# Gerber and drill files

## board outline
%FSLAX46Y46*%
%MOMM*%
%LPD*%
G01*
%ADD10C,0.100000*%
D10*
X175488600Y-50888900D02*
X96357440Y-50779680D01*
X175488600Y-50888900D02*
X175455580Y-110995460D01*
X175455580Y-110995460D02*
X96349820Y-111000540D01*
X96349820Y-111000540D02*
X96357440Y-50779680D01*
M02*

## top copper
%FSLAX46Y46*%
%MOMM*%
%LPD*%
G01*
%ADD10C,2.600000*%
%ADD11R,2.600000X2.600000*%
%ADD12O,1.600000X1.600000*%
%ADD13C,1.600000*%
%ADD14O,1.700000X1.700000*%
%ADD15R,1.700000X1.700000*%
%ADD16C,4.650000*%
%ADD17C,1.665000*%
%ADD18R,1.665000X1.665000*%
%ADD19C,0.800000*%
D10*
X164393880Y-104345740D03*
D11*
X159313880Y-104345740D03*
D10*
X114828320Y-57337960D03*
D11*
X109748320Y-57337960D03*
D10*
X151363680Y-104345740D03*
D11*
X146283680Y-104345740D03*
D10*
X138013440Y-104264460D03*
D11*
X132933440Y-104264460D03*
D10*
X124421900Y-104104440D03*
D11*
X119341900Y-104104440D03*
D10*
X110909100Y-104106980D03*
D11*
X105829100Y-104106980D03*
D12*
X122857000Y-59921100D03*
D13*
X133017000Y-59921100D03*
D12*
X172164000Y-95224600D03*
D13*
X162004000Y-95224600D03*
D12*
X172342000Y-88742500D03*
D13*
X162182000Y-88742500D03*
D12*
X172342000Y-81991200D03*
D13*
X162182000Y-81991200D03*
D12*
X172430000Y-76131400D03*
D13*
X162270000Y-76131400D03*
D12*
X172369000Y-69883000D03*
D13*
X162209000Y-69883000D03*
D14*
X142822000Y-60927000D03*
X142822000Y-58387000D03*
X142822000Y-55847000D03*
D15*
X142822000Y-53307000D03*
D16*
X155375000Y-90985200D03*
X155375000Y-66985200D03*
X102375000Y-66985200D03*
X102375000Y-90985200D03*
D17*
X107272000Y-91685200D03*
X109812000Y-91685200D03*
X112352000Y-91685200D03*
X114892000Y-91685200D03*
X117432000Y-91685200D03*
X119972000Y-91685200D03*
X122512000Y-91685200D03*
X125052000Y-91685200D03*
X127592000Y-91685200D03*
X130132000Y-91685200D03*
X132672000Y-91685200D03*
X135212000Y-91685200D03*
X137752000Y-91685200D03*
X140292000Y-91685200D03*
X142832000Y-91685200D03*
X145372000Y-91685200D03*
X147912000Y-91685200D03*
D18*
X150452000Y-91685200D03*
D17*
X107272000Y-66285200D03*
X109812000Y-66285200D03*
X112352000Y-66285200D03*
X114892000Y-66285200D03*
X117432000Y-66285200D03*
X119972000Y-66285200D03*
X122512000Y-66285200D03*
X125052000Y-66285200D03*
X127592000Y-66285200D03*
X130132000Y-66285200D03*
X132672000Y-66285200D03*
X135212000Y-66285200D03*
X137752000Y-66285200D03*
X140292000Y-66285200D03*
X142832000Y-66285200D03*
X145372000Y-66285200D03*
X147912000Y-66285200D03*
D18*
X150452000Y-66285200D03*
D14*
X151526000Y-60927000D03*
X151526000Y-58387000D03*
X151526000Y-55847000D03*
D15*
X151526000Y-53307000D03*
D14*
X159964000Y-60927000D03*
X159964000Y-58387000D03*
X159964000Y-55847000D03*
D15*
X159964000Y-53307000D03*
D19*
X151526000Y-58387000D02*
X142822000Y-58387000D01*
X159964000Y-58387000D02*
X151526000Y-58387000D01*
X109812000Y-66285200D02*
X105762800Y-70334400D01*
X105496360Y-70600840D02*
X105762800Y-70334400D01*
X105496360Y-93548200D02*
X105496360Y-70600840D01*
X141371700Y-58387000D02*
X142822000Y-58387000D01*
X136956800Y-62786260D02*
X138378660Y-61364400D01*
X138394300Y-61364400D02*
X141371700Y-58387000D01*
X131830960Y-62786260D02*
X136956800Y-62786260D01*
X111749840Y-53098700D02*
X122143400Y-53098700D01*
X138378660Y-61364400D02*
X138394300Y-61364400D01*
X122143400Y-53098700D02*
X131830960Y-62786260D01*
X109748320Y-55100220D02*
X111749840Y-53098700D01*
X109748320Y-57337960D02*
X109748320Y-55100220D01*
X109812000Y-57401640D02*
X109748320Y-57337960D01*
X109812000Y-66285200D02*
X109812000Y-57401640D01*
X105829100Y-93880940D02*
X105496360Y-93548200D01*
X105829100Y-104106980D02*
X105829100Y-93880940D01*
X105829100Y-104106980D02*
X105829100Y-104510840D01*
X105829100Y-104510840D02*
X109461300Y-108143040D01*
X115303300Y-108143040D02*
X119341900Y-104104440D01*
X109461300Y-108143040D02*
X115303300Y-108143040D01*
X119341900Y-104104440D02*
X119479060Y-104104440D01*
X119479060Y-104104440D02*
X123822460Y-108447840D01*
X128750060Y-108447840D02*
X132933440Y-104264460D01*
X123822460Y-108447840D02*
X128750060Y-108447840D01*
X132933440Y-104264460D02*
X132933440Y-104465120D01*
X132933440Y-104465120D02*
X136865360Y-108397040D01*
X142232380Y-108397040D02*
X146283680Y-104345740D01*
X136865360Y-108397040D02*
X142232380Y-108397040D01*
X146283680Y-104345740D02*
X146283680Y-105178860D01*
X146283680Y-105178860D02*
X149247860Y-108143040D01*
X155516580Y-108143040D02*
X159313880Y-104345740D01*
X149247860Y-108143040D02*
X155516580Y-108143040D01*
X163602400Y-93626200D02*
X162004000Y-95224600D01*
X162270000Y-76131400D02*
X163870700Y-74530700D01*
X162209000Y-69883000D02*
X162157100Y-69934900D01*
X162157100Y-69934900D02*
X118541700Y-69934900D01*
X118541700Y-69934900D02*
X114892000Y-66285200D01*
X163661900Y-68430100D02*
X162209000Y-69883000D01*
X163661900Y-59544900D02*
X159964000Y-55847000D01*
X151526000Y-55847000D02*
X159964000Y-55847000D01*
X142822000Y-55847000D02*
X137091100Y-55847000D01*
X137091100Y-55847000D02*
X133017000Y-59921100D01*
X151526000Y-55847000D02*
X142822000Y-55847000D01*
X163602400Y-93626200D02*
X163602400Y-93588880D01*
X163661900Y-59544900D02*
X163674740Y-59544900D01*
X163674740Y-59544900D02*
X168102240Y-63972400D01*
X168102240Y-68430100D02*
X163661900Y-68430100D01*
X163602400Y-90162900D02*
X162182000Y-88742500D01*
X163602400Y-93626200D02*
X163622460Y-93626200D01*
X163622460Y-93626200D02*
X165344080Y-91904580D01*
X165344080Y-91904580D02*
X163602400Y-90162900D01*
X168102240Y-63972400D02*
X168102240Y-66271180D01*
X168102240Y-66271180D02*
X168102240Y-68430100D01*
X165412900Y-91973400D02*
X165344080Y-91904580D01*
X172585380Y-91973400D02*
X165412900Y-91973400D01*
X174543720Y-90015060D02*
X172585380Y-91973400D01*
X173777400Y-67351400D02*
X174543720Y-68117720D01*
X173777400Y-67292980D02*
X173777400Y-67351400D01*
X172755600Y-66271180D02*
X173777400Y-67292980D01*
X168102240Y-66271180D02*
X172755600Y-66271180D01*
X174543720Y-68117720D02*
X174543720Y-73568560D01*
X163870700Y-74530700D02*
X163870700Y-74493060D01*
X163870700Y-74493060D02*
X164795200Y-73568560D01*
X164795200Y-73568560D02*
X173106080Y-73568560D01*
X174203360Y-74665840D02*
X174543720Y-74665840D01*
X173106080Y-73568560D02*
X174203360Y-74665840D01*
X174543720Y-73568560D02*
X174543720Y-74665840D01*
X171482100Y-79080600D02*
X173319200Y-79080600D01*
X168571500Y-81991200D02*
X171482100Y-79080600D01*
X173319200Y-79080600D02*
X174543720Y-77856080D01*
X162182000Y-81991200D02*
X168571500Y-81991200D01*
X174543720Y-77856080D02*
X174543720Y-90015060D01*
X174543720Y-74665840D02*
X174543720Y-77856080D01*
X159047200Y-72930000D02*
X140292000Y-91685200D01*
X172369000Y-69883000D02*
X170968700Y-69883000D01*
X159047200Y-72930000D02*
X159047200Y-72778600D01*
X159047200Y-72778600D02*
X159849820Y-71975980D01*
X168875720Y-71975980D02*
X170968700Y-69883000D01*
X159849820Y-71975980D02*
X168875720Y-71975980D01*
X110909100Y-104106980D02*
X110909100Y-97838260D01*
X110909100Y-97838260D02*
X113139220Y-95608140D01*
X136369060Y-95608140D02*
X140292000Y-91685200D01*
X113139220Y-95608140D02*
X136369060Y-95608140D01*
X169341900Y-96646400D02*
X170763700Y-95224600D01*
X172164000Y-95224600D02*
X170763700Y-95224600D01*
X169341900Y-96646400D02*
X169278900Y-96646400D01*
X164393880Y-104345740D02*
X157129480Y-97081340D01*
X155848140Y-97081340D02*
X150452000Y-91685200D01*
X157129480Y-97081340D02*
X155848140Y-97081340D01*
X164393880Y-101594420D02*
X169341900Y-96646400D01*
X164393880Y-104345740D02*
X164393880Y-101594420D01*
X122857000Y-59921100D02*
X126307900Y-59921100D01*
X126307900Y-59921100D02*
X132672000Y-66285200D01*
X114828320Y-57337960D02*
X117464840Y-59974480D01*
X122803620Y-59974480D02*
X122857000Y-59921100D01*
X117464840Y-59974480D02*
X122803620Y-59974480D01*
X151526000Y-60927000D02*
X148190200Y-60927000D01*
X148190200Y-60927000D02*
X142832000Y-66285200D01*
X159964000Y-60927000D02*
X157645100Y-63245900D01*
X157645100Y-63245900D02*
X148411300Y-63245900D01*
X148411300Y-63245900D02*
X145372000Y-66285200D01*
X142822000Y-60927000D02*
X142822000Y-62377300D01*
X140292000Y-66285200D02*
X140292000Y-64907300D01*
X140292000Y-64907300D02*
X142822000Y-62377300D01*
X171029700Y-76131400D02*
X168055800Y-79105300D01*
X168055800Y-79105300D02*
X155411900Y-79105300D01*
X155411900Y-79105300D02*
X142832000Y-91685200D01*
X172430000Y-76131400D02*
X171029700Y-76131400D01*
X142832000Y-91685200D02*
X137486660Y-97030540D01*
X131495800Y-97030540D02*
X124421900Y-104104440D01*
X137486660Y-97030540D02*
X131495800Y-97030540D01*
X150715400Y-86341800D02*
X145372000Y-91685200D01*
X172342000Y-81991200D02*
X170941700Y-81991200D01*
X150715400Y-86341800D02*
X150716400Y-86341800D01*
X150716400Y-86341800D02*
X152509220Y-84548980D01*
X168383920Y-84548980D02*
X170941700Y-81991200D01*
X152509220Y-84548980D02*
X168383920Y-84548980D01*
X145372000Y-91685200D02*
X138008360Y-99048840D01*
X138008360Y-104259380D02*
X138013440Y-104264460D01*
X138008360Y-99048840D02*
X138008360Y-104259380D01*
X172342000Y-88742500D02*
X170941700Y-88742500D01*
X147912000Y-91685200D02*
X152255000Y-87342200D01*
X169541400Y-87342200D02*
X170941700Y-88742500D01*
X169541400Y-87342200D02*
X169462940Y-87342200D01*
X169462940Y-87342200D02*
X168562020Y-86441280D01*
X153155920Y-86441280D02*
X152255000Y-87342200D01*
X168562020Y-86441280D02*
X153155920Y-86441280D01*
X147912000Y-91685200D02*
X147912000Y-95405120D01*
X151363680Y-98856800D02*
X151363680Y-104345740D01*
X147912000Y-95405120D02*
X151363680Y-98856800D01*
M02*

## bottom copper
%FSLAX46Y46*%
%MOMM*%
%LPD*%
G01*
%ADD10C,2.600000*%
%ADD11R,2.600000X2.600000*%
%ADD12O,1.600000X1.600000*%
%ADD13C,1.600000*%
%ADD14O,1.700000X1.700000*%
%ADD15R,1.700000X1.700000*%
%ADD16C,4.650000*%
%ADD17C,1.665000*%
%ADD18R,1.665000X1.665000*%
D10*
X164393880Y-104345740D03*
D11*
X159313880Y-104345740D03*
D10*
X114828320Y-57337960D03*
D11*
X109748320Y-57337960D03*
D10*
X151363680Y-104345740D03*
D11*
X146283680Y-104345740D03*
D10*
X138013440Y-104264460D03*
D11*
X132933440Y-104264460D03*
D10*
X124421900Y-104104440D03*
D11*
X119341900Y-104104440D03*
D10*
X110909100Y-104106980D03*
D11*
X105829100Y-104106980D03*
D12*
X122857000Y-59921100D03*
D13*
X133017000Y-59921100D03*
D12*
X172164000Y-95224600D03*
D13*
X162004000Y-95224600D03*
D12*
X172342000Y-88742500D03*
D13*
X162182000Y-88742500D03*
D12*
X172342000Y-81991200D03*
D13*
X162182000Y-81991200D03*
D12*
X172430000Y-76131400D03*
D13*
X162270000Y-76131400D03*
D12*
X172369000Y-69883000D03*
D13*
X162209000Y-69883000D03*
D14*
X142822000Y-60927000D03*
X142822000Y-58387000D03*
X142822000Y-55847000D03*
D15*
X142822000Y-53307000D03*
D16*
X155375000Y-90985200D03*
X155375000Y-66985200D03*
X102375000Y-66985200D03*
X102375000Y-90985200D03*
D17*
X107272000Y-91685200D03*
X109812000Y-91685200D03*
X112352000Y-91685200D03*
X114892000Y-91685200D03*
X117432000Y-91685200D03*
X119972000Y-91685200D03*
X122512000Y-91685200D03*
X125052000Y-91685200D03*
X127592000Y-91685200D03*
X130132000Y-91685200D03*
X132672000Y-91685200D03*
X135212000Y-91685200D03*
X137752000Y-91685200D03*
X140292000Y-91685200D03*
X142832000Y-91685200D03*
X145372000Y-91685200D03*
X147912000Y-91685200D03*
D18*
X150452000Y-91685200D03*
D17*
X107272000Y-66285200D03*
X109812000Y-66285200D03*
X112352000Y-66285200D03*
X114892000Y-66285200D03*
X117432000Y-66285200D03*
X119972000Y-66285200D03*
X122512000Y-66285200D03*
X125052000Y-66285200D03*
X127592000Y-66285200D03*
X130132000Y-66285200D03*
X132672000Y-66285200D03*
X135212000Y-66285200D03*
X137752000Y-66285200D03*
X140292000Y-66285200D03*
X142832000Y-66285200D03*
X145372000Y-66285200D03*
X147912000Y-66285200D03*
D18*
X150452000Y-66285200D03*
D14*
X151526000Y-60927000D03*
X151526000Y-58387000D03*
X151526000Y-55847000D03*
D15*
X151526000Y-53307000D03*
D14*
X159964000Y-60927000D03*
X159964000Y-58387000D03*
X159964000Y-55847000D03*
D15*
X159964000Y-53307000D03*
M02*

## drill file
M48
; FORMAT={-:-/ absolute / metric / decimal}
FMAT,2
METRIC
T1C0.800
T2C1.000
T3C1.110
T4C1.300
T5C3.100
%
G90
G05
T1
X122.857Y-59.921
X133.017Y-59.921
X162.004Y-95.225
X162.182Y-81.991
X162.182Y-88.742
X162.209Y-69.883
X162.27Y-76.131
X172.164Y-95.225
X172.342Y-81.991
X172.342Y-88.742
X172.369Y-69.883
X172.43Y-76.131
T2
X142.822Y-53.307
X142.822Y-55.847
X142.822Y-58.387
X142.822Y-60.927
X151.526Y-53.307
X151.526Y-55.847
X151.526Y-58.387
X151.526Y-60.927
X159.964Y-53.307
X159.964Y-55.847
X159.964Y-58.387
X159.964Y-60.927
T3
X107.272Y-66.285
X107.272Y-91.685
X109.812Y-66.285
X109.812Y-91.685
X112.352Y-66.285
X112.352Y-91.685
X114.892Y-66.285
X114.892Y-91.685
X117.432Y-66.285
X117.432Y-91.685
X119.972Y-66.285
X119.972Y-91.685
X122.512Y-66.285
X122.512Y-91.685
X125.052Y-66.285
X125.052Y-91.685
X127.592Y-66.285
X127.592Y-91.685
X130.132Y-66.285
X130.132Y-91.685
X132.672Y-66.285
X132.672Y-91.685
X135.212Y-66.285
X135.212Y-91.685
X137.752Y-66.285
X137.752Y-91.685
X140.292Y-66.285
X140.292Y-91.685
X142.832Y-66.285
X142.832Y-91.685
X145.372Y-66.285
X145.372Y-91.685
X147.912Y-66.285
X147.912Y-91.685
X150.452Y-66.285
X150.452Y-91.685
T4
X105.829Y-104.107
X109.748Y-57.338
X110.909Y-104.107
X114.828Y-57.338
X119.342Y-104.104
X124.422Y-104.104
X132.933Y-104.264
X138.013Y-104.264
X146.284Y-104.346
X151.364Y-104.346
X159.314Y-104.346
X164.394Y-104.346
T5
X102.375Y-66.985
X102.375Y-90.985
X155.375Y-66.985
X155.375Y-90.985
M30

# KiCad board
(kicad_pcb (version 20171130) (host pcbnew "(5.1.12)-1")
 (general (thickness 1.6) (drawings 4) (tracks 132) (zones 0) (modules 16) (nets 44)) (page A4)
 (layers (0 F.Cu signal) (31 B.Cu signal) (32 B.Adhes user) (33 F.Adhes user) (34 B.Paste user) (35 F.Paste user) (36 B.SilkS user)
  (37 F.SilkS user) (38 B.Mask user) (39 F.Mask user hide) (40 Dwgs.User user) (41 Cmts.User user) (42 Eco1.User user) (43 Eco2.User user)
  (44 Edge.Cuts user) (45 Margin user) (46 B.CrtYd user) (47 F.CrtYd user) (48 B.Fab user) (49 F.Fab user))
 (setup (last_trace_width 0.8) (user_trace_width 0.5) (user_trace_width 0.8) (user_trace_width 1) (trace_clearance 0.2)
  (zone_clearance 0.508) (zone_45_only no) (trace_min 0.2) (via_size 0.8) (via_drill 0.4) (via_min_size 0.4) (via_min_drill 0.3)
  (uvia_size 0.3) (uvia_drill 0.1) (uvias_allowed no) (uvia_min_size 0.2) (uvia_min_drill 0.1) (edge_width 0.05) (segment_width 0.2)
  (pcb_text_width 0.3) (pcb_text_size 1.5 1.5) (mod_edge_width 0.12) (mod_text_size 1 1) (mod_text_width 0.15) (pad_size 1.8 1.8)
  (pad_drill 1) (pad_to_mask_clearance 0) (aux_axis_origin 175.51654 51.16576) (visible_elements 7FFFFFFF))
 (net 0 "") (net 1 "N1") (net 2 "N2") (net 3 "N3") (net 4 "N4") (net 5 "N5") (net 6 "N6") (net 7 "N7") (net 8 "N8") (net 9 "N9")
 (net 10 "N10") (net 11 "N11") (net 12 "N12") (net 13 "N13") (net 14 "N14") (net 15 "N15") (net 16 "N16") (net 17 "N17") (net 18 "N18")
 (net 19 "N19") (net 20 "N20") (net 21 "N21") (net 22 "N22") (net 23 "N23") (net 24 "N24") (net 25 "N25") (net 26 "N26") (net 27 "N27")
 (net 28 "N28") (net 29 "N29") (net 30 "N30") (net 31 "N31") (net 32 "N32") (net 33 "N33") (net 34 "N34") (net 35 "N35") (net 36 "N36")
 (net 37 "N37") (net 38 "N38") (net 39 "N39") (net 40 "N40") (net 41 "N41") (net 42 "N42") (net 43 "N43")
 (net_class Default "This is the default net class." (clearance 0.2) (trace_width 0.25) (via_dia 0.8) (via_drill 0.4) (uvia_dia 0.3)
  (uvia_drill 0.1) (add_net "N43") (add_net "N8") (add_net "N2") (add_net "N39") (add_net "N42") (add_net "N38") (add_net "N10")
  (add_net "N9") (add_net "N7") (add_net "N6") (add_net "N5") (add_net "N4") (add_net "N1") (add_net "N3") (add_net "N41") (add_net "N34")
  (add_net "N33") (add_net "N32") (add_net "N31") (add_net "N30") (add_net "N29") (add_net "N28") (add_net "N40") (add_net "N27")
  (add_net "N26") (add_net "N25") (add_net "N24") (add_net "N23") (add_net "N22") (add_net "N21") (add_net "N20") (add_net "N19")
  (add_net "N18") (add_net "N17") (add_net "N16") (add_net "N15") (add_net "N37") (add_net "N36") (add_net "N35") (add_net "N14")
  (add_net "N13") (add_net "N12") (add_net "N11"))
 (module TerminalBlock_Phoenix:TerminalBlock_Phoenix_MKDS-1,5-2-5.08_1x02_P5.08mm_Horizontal (layer F.Cu) (at 159.31388 104.34574)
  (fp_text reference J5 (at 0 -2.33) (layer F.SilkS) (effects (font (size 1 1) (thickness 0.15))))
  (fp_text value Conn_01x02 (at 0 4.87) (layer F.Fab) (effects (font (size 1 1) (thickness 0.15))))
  (pad 2 thru_hole circle (at 5.08 0) (size 2.6 2.6) (drill 1.3) (layers *.Cu *.Mask) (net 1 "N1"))
  (pad 1 thru_hole rect (at 0 0) (size 2.6 2.6) (drill 1.3) (layers *.Cu *.Mask) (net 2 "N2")))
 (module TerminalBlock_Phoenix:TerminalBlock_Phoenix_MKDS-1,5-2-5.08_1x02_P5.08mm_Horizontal (layer F.Cu) (at 109.74832 57.33796)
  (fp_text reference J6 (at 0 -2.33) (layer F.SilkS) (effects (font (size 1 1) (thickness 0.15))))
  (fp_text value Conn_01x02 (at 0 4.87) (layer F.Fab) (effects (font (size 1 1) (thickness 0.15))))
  (pad 2 thru_hole circle (at 5.08 0) (size 2.6 2.6) (drill 1.3) (layers *.Cu *.Mask) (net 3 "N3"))
  (pad 1 thru_hole rect (at 0 0) (size 2.6 2.6) (drill 1.3) (layers *.Cu *.Mask) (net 2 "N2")))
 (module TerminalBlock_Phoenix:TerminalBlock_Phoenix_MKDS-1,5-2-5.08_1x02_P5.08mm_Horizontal (layer F.Cu) (at 146.28368 104.34574)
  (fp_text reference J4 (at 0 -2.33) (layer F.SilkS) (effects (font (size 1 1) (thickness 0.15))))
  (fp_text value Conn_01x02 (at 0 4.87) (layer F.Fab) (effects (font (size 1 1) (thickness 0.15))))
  (pad 2 thru_hole circle (at 5.08 0) (size 2.6 2.6) (drill 1.3) (layers *.Cu *.Mask) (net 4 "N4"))
  (pad 1 thru_hole rect (at 0 0) (size 2.6 2.6) (drill 1.3) (layers *.Cu *.Mask) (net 2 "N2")))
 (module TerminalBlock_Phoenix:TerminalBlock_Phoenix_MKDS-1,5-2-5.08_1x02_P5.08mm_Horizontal (layer F.Cu) (at 132.93344 104.26446)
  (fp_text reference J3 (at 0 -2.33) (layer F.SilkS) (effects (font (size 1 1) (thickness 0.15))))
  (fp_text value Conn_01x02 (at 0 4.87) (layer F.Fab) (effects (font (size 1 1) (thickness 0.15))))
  (pad 2 thru_hole circle (at 5.08 0) (size 2.6 2.6) (drill 1.3) (layers *.Cu *.Mask) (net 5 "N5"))
  (pad 1 thru_hole rect (at 0 0) (size 2.6 2.6) (drill 1.3) (layers *.Cu *.Mask) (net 2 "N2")))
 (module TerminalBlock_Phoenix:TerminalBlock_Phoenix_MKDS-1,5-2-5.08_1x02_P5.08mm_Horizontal (layer F.Cu) (at 119.3419 104.10444)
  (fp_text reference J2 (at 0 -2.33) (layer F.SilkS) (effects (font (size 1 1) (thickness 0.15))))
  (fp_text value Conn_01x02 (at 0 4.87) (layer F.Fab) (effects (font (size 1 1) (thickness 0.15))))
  (pad 2 thru_hole circle (at 5.08 0) (size 2.6 2.6) (drill 1.3) (layers *.Cu *.Mask) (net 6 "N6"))
  (pad 1 thru_hole rect (at 0 0) (size 2.6 2.6) (drill 1.3) (layers *.Cu *.Mask) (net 2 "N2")))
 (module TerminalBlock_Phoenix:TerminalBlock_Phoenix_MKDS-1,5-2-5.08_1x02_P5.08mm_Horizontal (layer F.Cu) (at 105.8291 104.10698)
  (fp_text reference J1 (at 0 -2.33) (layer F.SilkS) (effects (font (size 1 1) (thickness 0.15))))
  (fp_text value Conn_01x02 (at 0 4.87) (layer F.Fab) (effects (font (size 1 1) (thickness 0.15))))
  (pad 2 thru_hole circle (at 5.08 0) (size 2.6 2.6) (drill 1.3) (layers *.Cu *.Mask) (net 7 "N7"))
  (pad 1 thru_hole rect (at 0 0) (size 2.6 2.6) (drill 1.3) (layers *.Cu *.Mask) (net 2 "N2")))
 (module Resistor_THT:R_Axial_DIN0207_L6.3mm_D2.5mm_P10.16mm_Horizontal (layer F.Cu) (at 133.017 59.9211 180)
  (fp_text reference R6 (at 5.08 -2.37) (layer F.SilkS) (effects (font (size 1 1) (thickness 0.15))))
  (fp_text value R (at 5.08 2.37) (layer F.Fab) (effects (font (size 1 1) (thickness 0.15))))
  (pad 2 thru_hole oval (at 10.16 0 180) (size 1.6 1.6) (drill 0.8) (layers *.Cu *.Mask) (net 3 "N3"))
  (pad 1 thru_hole circle (at 0 0 180) (size 1.6 1.6) (drill 0.8) (layers *.Cu *.Mask) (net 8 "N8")))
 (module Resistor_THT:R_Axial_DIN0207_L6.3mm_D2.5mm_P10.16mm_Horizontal (layer F.Cu) (at 162.004 95.2246)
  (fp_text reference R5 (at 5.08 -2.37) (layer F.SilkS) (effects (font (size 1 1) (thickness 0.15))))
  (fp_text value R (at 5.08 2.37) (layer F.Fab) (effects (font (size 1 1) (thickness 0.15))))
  (pad 2 thru_hole oval (at 10.16 0) (size 1.6 1.6) (drill 0.8) (layers *.Cu *.Mask) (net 1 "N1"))
  (pad 1 thru_hole circle (at 0 0) (size 1.6 1.6) (drill 0.8) (layers *.Cu *.Mask) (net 8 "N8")))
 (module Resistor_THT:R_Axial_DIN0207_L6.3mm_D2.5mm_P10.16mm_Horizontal (layer F.Cu) (at 162.182 88.7425)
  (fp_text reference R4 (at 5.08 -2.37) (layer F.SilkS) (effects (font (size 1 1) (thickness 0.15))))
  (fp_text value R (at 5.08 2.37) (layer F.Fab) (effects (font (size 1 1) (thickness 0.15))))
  (pad 2 thru_hole oval (at 10.16 0) (size 1.6 1.6) (drill 0.8) (layers *.Cu *.Mask) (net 4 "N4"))
  (pad 1 thru_hole circle (at 0 0) (size 1.6 1.6) (drill 0.8) (layers *.Cu *.Mask) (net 8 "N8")))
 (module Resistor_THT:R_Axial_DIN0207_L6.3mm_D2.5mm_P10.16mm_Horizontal (layer F.Cu) (at 162.182 81.9912)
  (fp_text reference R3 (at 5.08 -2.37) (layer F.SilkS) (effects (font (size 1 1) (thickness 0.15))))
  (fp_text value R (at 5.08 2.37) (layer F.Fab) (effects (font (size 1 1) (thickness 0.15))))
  (pad 2 thru_hole oval (at 10.16 0) (size 1.6 1.6) (drill 0.8) (layers *.Cu *.Mask) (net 5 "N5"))
  (pad 1 thru_hole circle (at 0 0) (size 1.6 1.6) (drill 0.8) (layers *.Cu *.Mask) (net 8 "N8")))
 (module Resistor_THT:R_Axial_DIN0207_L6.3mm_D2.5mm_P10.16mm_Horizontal (layer F.Cu) (at 162.27 76.1314)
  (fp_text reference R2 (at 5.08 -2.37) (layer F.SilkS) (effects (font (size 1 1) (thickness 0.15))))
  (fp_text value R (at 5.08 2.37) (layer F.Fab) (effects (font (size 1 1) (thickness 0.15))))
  (pad 2 thru_hole oval (at 10.16 0) (size 1.6 1.6) (drill 0.8) (layers *.Cu *.Mask) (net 6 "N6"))
  (pad 1 thru_hole circle (at 0 0) (size 1.6 1.6) (drill 0.8) (layers *.Cu *.Mask) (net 8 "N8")))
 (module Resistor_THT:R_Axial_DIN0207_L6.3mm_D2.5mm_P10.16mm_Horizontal (layer F.Cu) (at 162.209 69.883)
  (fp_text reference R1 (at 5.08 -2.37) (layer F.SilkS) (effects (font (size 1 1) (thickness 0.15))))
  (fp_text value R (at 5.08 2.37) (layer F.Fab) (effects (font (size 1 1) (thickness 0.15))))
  (pad 2 thru_hole oval (at 10.16 0) (size 1.6 1.6) (drill 0.8) (layers *.Cu *.Mask) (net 7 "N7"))
  (pad 1 thru_hole circle (at 0 0) (size 1.6 1.6) (drill 0.8) (layers *.Cu *.Mask) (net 8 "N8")))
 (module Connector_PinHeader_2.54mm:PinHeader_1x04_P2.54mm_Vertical (layer F.Cu) (at 142.822 53.307)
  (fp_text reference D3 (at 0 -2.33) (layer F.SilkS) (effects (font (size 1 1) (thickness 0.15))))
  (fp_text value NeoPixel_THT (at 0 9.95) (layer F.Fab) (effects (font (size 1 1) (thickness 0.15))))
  (pad 4 thru_hole oval (at 0 7.62) (size 1.7 1.7) (drill 1) (layers *.Cu *.Mask) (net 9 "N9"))
  (pad 3 thru_hole oval (at 0 5.08) (size 1.7 1.7) (drill 1) (layers *.Cu *.Mask) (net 2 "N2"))
  (pad 2 thru_hole oval (at 0 2.54) (size 1.7 1.7) (drill 1) (layers *.Cu *.Mask) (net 8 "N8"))
  (pad 1 thru_hole rect (at 0 0) (size 1.7 1.7) (drill 1) (layers *.Cu *.Mask) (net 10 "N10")))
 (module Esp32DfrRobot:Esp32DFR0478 (layer F.Cu) (at 125.052 78.9852)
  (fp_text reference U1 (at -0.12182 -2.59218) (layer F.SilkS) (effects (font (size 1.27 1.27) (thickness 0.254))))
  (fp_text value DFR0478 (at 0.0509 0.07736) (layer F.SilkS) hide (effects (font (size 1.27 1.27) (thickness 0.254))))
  (pad MH4 thru_hole circle (at 30.323 12) (size 4.65 4.65) (drill 3.1) (layers *.Cu *.Mask) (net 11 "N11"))
  (pad MH3 thru_hole circle (at 30.323 -12) (size 4.65 4.65) (drill 3.1) (layers *.Cu *.Mask) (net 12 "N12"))
  (pad MH2 thru_hole circle (at -22.677 -12) (size 4.65 4.65) (drill 3.1) (layers *.Cu *.Mask) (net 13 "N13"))
  (pad MH1 thru_hole circle (at -22.677 12) (size 4.65 4.65) (drill 3.1) (layers *.Cu *.Mask) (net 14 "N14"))
  (pad 36 thru_hole circle (at -17.78 12.7) (size 1.665 1.665) (drill 1.11) (layers *.Cu *.Mask) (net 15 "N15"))
  (pad 35 thru_hole circle (at -15.24 12.7) (size 1.665 1.665) (drill 1.11) (layers *.Cu *.Mask) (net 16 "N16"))
  (pad 34 thru_hole circle (at -12.7 12.7) (size 1.665 1.665) (drill 1.11) (layers *.Cu *.Mask) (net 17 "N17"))
  (pad 33 thru_hole circle (at -10.16 12.7) (size 1.665 1.665) (drill 1.11) (layers *.Cu *.Mask) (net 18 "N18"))
  (pad 32 thru_hole circle (at -7.62 12.7) (size 1.665 1.665) (drill 1.11) (layers *.Cu *.Mask) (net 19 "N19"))
  (pad 31 thru_hole circle (at -5.08 12.7) (size 1.665 1.665) (drill 1.11) (layers *.Cu *.Mask) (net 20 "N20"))
  (pad 30 thru_hole circle (at -2.54 12.7) (size 1.665 1.665) (drill 1.11) (layers *.Cu *.Mask) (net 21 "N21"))
  (pad 29 thru_hole circle (at 0 12.7) (size 1.665 1.665) (drill 1.11) (layers *.Cu *.Mask) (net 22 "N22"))
  (pad 28 thru_hole circle (at 2.54 12.7) (size 1.665 1.665) (drill 1.11) (layers *.Cu *.Mask) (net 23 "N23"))
  (pad 27 thru_hole circle (at 5.08 12.7) (size 1.665 1.665) (drill 1.11) (layers *.Cu *.Mask) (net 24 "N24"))
  (pad 26 thru_hole circle (at 7.62 12.7) (size 1.665 1.665) (drill 1.11) (layers *.Cu *.Mask) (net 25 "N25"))
  (pad 25 thru_hole circle (at 10.16 12.7) (size 1.665 1.665) (drill 1.11) (layers *.Cu *.Mask) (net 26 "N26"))
  (pad 24 thru_hole circle (at 12.7 12.7) (size 1.665 1.665) (drill 1.11) (layers *.Cu *.Mask) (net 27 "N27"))
  (pad 23 thru_hole circle (at 15.24 12.7) (size 1.665 1.665) (drill 1.11) (layers *.Cu *.Mask) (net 7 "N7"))
  (pad 22 thru_hole circle (at 17.78 12.7) (size 1.665 1.665) (drill 1.11) (layers *.Cu *.Mask) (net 6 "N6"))
  (pad 21 thru_hole circle (at 20.32 12.7) (size 1.665 1.665) (drill 1.11) (layers *.Cu *.Mask) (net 5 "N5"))
  (pad 20 thru_hole circle (at 22.86 12.7) (size 1.665 1.665) (drill 1.11) (layers *.Cu *.Mask) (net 4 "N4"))
  (pad 19 thru_hole rect (at 25.4 12.7) (size 1.665 1.665) (drill 1.11) (layers *.Cu *.Mask) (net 1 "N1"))
  (pad 18 thru_hole circle (at -17.78 -12.7) (size 1.665 1.665) (drill 1.11) (layers *.Cu *.Mask) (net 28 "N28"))
  (pad 17 thru_hole circle (at -15.24 -12.7) (size 1.665 1.665) (drill 1.11) (layers *.Cu *.Mask) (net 2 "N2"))
  (pad 16 thru_hole circle (at -12.7 -12.7) (size 1.665 1.665) (drill 1.11) (layers *.Cu *.Mask) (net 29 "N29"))
  (pad 15 thru_hole circle (at -10.16 -12.7) (size 1.665 1.665) (drill 1.11) (layers *.Cu *.Mask) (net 8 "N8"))
  (pad 14 thru_hole circle (at -7.62 -12.7) (size 1.665 1.665) (drill 1.11) (layers *.Cu *.Mask) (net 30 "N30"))
  (pad 13 thru_hole circle (at -5.08 -12.7) (size 1.665 1.665) (drill 1.11) (layers *.Cu *.Mask) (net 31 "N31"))
  (pad 12 thru_hole circle (at -2.54 -12.7) (size 1.665 1.665) (drill 1.11) (layers *.Cu *.Mask) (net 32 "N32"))
  (pad 11 thru_hole circle (at 0 -12.7) (size 1.665 1.665) (drill 1.11) (layers *.Cu *.Mask) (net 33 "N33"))
  (pad 10 thru_hole circle (at 2.54 -12.7) (size 1.665 1.665) (drill 1.11) (layers *.Cu *.Mask) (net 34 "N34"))
  (pad 9 thru_hole circle (at 5.08 -12.7) (size 1.665 1.665) (drill 1.11) (layers *.Cu *.Mask) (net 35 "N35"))
  (pad 8 thru_hole circle (at 7.62 -12.7) (size 1.665 1.665) (drill 1.11) (layers *.Cu *.Mask) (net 3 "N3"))
  (pad 7 thru_hole circle (at 10.16 -12.7) (size 1.665 1.665) (drill 1.11) (layers *.Cu *.Mask) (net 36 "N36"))
  (pad 6 thru_hole circle (at 12.7 -12.7) (size 1.665 1.665) (drill 1.11) (layers *.Cu *.Mask) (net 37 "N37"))
  (pad 5 thru_hole circle (at 15.24 -12.7) (size 1.665 1.665) (drill 1.11) (layers *.Cu *.Mask) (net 9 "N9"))
  (pad 4 thru_hole circle (at 17.78 -12.7) (size 1.665 1.665) (drill 1.11) (layers *.Cu *.Mask) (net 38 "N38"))
  (pad 3 thru_hole circle (at 20.32 -12.7) (size 1.665 1.665) (drill 1.11) (layers *.Cu *.Mask) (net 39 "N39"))
  (pad 2 thru_hole circle (at 22.86 -12.7) (size 1.665 1.665) (drill 1.11) (layers *.Cu *.Mask) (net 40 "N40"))
  (pad 1 thru_hole rect (at 25.4 -12.7) (size 1.665 1.665) (drill 1.11) (layers *.Cu *.Mask) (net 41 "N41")))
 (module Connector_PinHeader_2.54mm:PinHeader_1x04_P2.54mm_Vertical (layer F.Cu) (at 151.526 53.307)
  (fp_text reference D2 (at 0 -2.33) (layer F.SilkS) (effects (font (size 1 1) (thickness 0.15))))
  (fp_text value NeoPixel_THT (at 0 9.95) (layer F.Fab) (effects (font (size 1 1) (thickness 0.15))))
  (pad 4 thru_hole oval (at 0 7.62) (size 1.7 1.7) (drill 1) (layers *.Cu *.Mask) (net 38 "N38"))
  (pad 3 thru_hole oval (at 0 5.08) (size 1.7 1.7) (drill 1) (layers *.Cu *.Mask) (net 2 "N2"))
  (pad 2 thru_hole oval (at 0 2.54) (size 1.7 1.7) (drill 1) (layers *.Cu *.Mask) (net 8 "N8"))
  (pad 1 thru_hole rect (at 0 0) (size 1.7 1.7) (drill 1) (layers *.Cu *.Mask) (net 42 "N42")))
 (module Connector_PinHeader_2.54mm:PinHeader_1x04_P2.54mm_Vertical (layer F.Cu) (at 159.964 53.307)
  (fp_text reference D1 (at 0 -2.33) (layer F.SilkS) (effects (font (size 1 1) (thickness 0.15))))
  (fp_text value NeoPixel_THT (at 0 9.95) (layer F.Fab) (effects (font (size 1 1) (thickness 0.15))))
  (pad 4 thru_hole oval (at 0 7.62) (size 1.7 1.7) (drill 1) (layers *.Cu *.Mask) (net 39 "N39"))
  (pad 3 thru_hole oval (at 0 5.08) (size 1.7 1.7) (drill 1) (layers *.Cu *.Mask) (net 2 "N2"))
  (pad 2 thru_hole oval (at 0 2.54) (size 1.7 1.7) (drill 1) (layers *.Cu *.Mask) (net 8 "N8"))
  (pad 1 thru_hole rect (at 0 0) (size 1.7 1.7) (drill 1) (layers *.Cu *.Mask) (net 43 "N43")))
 (gr_line (start 175.4886 50.8889) (end 96.35744 50.77968) (layer Edge.Cuts) (width 0.1))
 (gr_line (start 175.4886 50.8889) (end 175.45558 110.99546) (layer Edge.Cuts) (width 0.1))
 (gr_line (start 175.45558 110.99546) (end 96.34982 111.00054) (layer Edge.Cuts) (width 0.1))
 (gr_line (start 96.34982 111.00054) (end 96.35744 50.77968) (layer Edge.Cuts) (width 0.1))
 (segment (start 151.526 58.387) (end 142.822 58.387) (width 0.8) (layer F.Cu) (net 2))
 (segment (start 159.964 58.387) (end 151.526 58.387) (width 0.8) (layer F.Cu) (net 2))
 (segment (start 109.812 66.2852) (end 105.7628 70.3344) (width 0.8) (layer F.Cu) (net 2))
 (segment (start 105.49636 70.60084) (end 105.7628 70.3344) (width 0.8) (layer F.Cu) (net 2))
 (segment (start 105.49636 93.5482) (end 105.49636 70.60084) (width 0.8) (layer F.Cu) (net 2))
 (segment (start 141.3717 58.387) (end 142.822 58.387) (width 0.8) (layer F.Cu) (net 2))
 (segment (start 136.9568 62.78626) (end 138.37866 61.3644) (width 0.8) (layer F.Cu) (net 2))
 (segment (start 138.3943 61.3644) (end 141.3717 58.387) (width 0.8) (layer F.Cu) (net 2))
 (segment (start 131.83096 62.78626) (end 136.9568 62.78626) (width 0.8) (layer F.Cu) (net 2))
 (segment (start 111.74984 53.0987) (end 122.1434 53.0987) (width 0.8) (layer F.Cu) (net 2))
 (segment (start 138.37866 61.3644) (end 138.3943 61.3644) (width 0.8) (layer F.Cu) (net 2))
 (segment (start 122.1434 53.0987) (end 131.83096 62.78626) (width 0.8) (layer F.Cu) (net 2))
 (segment (start 109.74832 55.10022) (end 111.74984 53.0987) (width 0.8) (layer F.Cu) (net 2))
 (segment (start 109.74832 57.33796) (end 109.74832 55.10022) (width 0.8) (layer F.Cu) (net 2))
 (segment (start 109.812 57.40164) (end 109.74832 57.33796) (width 0.8) (layer F.Cu) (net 2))
 (segment (start 109.812 66.2852) (end 109.812 57.40164) (width 0.8) (layer F.Cu) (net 2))
 (segment (start 105.8291 93.88094) (end 105.49636 93.5482) (width 0.8) (layer F.Cu) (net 2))
 (segment (start 105.8291 104.10698) (end 105.8291 93.88094) (width 0.8) (layer F.Cu) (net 2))
 (segment (start 105.8291 104.10698) (end 105.8291 104.51084) (width 0.8) (layer F.Cu) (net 2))
 (segment (start 105.8291 104.51084) (end 109.4613 108.14304) (width 0.8) (layer F.Cu) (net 2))
 (segment (start 115.3033 108.14304) (end 119.3419 104.10444) (width 0.8) (layer F.Cu) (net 2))
 (segment (start 109.4613 108.14304) (end 115.3033 108.14304) (width 0.8) (layer F.Cu) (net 2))
 (segment (start 119.3419 104.10444) (end 119.47906 104.10444) (width 0.8) (layer F.Cu) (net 2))
 (segment (start 119.47906 104.10444) (end 123.82246 108.44784) (width 0.8) (layer F.Cu) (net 2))
 (segment (start 128.75006 108.44784) (end 132.93344 104.26446) (width 0.8) (layer F.Cu) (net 2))
 (segment (start 123.82246 108.44784) (end 128.75006 108.44784) (width 0.8) (layer F.Cu) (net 2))
 (segment (start 132.93344 104.26446) (end 132.93344 104.46512) (width 0.8) (layer F.Cu) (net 2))
 (segment (start 132.93344 104.46512) (end 136.86536 108.39704) (width 0.8) (layer F.Cu) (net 2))
 (segment (start 142.23238 108.39704) (end 146.28368 104.34574) (width 0.8) (layer F.Cu) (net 2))
 (segment (start 136.86536 108.39704) (end 142.23238 108.39704) (width 0.8) (layer F.Cu) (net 2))
 (segment (start 146.28368 104.34574) (end 146.28368 105.17886) (width 0.8) (layer F.Cu) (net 2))
 (segment (start 146.28368 105.17886) (end 149.24786 108.14304) (width 0.8) (layer F.Cu) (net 2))
 (segment (start 155.51658 108.14304) (end 159.31388 104.34574) (width 0.8) (layer F.Cu) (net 2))
 (segment (start 149.24786 108.14304) (end 155.51658 108.14304) (width 0.8) (layer F.Cu) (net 2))
 (segment (start 163.6024 93.6262) (end 162.004 95.2246) (width 0.8) (layer F.Cu) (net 8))
 (segment (start 162.27 76.1314) (end 163.8707 74.5307) (width 0.8) (layer F.Cu) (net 8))
 (segment (start 162.209 69.883) (end 162.1571 69.9349) (width 0.8) (layer F.Cu) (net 8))
 (segment (start 162.1571 69.9349) (end 118.5417 69.9349) (width 0.8) (layer F.Cu) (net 8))
 (segment (start 118.5417 69.9349) (end 114.892 66.2852) (width 0.8) (layer F.Cu) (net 8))
 (segment (start 163.6619 68.4301) (end 162.209 69.883) (width 0.8) (layer F.Cu) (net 8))
 (segment (start 163.6619 59.5449) (end 159.964 55.847) (width 0.8) (layer F.Cu) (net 8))
 (segment (start 151.526 55.847) (end 159.964 55.847) (width 0.8) (layer F.Cu) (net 8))
 (segment (start 142.822 55.847) (end 137.0911 55.847) (width 0.8) (layer F.Cu) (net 8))
 (segment (start 137.0911 55.847) (end 133.017 59.9211) (width 0.8) (layer F.Cu) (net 8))
 (segment (start 151.526 55.847) (end 142.822 55.847) (width 0.8) (layer F.Cu) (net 8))
 (segment (start 163.6024 93.6262) (end 163.6024 93.58888) (width 0.8) (layer F.Cu) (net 8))
 (segment (start 163.6619 59.5449) (end 163.67474 59.5449) (width 0.8) (layer F.Cu) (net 8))
 (segment (start 163.67474 59.5449) (end 168.10224 63.9724) (width 0.8) (layer F.Cu) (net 8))
 (segment (start 168.10224 68.4301) (end 163.6619 68.4301) (width 0.8) (layer F.Cu) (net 8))
 (segment (start 163.6024 90.1629) (end 162.182 88.7425) (width 0.8) (layer F.Cu) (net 8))
 (segment (start 163.6024 93.6262) (end 163.62246 93.6262) (width 0.8) (layer F.Cu) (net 8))
 (segment (start 163.62246 93.6262) (end 165.34408 91.90458) (width 0.8) (layer F.Cu) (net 8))
 (segment (start 165.34408 91.90458) (end 163.6024 90.1629) (width 0.8) (layer F.Cu) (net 8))
 (segment (start 168.10224 63.9724) (end 168.10224 66.27118) (width 0.8) (layer F.Cu) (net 8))
 (segment (start 168.10224 66.27118) (end 168.10224 68.4301) (width 0.8) (layer F.Cu) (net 8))
 (segment (start 165.4129 91.9734) (end 165.34408 91.90458) (width 0.8) (layer F.Cu) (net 8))
 (segment (start 172.58538 91.9734) (end 165.4129 91.9734) (width 0.8) (layer F.Cu) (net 8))
 (segment (start 174.54372 90.01506) (end 172.58538 91.9734) (width 0.8) (layer F.Cu) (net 8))
 (segment (start 173.7774 67.3514) (end 174.54372 68.11772) (width 0.8) (layer F.Cu) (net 8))
 (segment (start 173.7774 67.29298) (end 173.7774 67.3514) (width 0.8) (layer F.Cu) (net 8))
 (segment (start 172.7556 66.27118) (end 173.7774 67.29298) (width 0.8) (layer F.Cu) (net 8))
 (segment (start 168.10224 66.27118) (end 172.7556 66.27118) (width 0.8) (layer F.Cu) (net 8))
 (segment (start 174.54372 68.11772) (end 174.54372 73.56856) (width 0.8) (layer F.Cu) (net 8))
 (segment (start 163.8707 74.5307) (end 163.8707 74.49306) (width 0.8) (layer F.Cu) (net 8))
 (segment (start 163.8707 74.49306) (end 164.7952 73.56856) (width 0.8) (layer F.Cu) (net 8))
 (segment (start 164.7952 73.56856) (end 173.10608 73.56856) (width 0.8) (layer F.Cu) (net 8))
 (segment (start 174.20336 74.66584) (end 174.54372 74.66584) (width 0.8) (layer F.Cu) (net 8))
 (segment (start 173.10608 73.56856) (end 174.20336 74.66584) (width 0.8) (layer F.Cu) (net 8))
 (segment (start 174.54372 73.56856) (end 174.54372 74.66584) (width 0.8) (layer F.Cu) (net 8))
 (segment (start 171.4821 79.0806) (end 173.3192 79.0806) (width 0.8) (layer F.Cu) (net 8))
 (segment (start 168.5715 81.9912) (end 171.4821 79.0806) (width 0.8) (layer F.Cu) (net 8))
 (segment (start 173.3192 79.0806) (end 174.54372 77.85608) (width 0.8) (layer F.Cu) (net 8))
 (segment (start 162.182 81.9912) (end 168.5715 81.9912) (width 0.8) (layer F.Cu) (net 8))
 (segment (start 174.54372 77.85608) (end 174.54372 90.01506) (width 0.8) (layer F.Cu) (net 8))
 (segment (start 174.54372 74.66584) (end 174.54372 77.85608) (width 0.8) (layer F.Cu) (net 8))
 (segment (start 159.0472 72.93) (end 140.292 91.6852) (width 0.8) (layer F.Cu) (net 7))
 (segment (start 172.369 69.883) (end 170.9687 69.883) (width 0.8) (layer F.Cu) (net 7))
 (segment (start 159.0472 72.93) (end 159.0472 72.7786) (width 0.8) (layer F.Cu) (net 7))
 (segment (start 159.0472 72.7786) (end 159.84982 71.97598) (width 0.8) (layer F.Cu) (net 7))
 (segment (start 168.87572 71.97598) (end 170.9687 69.883) (width 0.8) (layer F.Cu) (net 7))
 (segment (start 159.84982 71.97598) (end 168.87572 71.97598) (width 0.8) (layer F.Cu) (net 7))
 (segment (start 110.9091 104.10698) (end 110.9091 97.83826) (width 0.8) (layer F.Cu) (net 7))
 (segment (start 110.9091 97.83826) (end 113.13922 95.60814) (width 0.8) (layer F.Cu) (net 7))
 (segment (start 136.36906 95.60814) (end 140.292 91.6852) (width 0.8) (layer F.Cu) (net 7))
 (segment (start 113.13922 95.60814) (end 136.36906 95.60814) (width 0.8) (layer F.Cu) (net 7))
 (segment (start 169.3419 96.6464) (end 170.7637 95.2246) (width 0.8) (layer F.Cu) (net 1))
 (segment (start 172.164 95.2246) (end 170.7637 95.2246) (width 0.8) (layer F.Cu) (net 1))
 (segment (start 169.3419 96.6464) (end 169.2789 96.6464) (width 0.8) (layer F.Cu) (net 1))
 (segment (start 164.39388 104.34574) (end 157.12948 97.08134) (width 0.8) (layer F.Cu) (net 1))
 (segment (start 155.84814 97.08134) (end 150.452 91.6852) (width 0.8) (layer F.Cu) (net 1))
 (segment (start 157.12948 97.08134) (end 155.84814 97.08134) (width 0.8) (layer F.Cu) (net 1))
 (segment (start 164.39388 101.59442) (end 169.3419 96.6464) (width 0.8) (layer F.Cu) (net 1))
 (segment (start 164.39388 104.34574) (end 164.39388 101.59442) (width 0.8) (layer F.Cu) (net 1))
 (segment (start 122.857 59.9211) (end 126.3079 59.9211) (width 0.8) (layer F.Cu) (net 3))
 (segment (start 126.3079 59.9211) (end 132.672 66.2852) (width 0.8) (layer F.Cu) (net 3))
 (segment (start 114.82832 57.33796) (end 117.46484 59.97448) (width 0.8) (layer F.Cu) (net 3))
 (segment (start 122.80362 59.97448) (end 122.857 59.9211) (width 0.8) (layer F.Cu) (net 3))
 (segment (start 117.46484 59.97448) (end 122.80362 59.97448) (width 0.8) (layer F.Cu) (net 3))
 (segment (start 151.526 60.927) (end 148.1902 60.927) (width 0.8) (layer F.Cu) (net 38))
 (segment (start 148.1902 60.927) (end 142.832 66.2852) (width 0.8) (layer F.Cu) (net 38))
 (segment (start 159.964 60.927) (end 157.6451 63.2459) (width 0.8) (layer F.Cu) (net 39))
 (segment (start 157.6451 63.2459) (end 148.4113 63.2459) (width 0.8) (layer F.Cu) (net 39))
 (segment (start 148.4113 63.2459) (end 145.372 66.2852) (width 0.8) (layer F.Cu) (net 39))
 (segment (start 142.822 60.927) (end 142.822 62.3773) (width 0.8) (layer F.Cu) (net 9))
 (segment (start 140.292 66.2852) (end 140.292 64.9073) (width 0.8) (layer F.Cu) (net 9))
 (segment (start 140.292 64.9073) (end 142.822 62.3773) (width 0.8) (layer F.Cu) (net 9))
 (segment (start 171.0297 76.1314) (end 168.0558 79.1053) (width 0.8) (layer F.Cu) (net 6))
 (segment (start 168.0558 79.1053) (end 155.4119 79.1053) (width 0.8) (layer F.Cu) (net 6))
 (segment (start 155.4119 79.1053) (end 142.832 91.6852) (width 0.8) (layer F.Cu) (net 6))
 (segment (start 172.43 76.1314) (end 171.0297 76.1314) (width 0.8) (layer F.Cu) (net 6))
 (segment (start 142.832 91.6852) (end 137.48666 97.03054) (width 0.8) (layer F.Cu) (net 6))
 (segment (start 131.4958 97.03054) (end 124.4219 104.10444) (width 0.8) (layer F.Cu) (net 6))
 (segment (start 137.48666 97.03054) (end 131.4958 97.03054) (width 0.8) (layer F.Cu) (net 6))
 (segment (start 150.7154 86.3418) (end 145.372 91.6852) (width 0.8) (layer F.Cu) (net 5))
 (segment (start 172.342 81.9912) (end 170.9417 81.9912) (width 0.8) (layer F.Cu) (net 5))
 (segment (start 150.7154 86.3418) (end 150.7164 86.3418) (width 0.8) (layer F.Cu) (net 5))
 (segment (start 150.7164 86.3418) (end 152.50922 84.54898) (width 0.8) (layer F.Cu) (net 5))
 (segment (start 168.38392 84.54898) (end 170.9417 81.9912) (width 0.8) (layer F.Cu) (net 5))
 (segment (start 152.50922 84.54898) (end 168.38392 84.54898) (width 0.8) (layer F.Cu) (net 5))
 (segment (start 145.372 91.6852) (end 138.00836 99.04884) (width 0.8) (layer F.Cu) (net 5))
 (segment (start 138.00836 104.25938) (end 138.01344 104.26446) (width 0.8) (layer F.Cu) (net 5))
 (segment (start 138.00836 99.04884) (end 138.00836 104.25938) (width 0.8) (layer F.Cu) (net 5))
 (segment (start 172.342 88.7425) (end 170.9417 88.7425) (width 0.8) (layer F.Cu) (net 4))
 (segment (start 147.912 91.6852) (end 152.255 87.3422) (width 0.8) (layer F.Cu) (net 4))
 (segment (start 169.5414 87.3422) (end 170.9417 88.7425) (width 0.8) (layer F.Cu) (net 4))
 (segment (start 169.5414 87.3422) (end 169.46294 87.3422) (width 0.8) (layer F.Cu) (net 4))
 (segment (start 169.46294 87.3422) (end 168.56202 86.44128) (width 0.8) (layer F.Cu) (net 4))
 (segment (start 153.15592 86.44128) (end 152.255 87.3422) (width 0.8) (layer F.Cu) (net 4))
 (segment (start 168.56202 86.44128) (end 153.15592 86.44128) (width 0.8) (layer F.Cu) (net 4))
 (segment (start 147.912 91.6852) (end 147.912 95.40512) (width 0.8) (layer F.Cu) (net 4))
 (segment (start 151.36368 98.8568) (end 151.36368 104.34574) (width 0.8) (layer F.Cu) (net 4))
 (segment (start 147.912 95.40512) (end 151.36368 98.8568) (width 0.8) (layer F.Cu) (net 4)))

